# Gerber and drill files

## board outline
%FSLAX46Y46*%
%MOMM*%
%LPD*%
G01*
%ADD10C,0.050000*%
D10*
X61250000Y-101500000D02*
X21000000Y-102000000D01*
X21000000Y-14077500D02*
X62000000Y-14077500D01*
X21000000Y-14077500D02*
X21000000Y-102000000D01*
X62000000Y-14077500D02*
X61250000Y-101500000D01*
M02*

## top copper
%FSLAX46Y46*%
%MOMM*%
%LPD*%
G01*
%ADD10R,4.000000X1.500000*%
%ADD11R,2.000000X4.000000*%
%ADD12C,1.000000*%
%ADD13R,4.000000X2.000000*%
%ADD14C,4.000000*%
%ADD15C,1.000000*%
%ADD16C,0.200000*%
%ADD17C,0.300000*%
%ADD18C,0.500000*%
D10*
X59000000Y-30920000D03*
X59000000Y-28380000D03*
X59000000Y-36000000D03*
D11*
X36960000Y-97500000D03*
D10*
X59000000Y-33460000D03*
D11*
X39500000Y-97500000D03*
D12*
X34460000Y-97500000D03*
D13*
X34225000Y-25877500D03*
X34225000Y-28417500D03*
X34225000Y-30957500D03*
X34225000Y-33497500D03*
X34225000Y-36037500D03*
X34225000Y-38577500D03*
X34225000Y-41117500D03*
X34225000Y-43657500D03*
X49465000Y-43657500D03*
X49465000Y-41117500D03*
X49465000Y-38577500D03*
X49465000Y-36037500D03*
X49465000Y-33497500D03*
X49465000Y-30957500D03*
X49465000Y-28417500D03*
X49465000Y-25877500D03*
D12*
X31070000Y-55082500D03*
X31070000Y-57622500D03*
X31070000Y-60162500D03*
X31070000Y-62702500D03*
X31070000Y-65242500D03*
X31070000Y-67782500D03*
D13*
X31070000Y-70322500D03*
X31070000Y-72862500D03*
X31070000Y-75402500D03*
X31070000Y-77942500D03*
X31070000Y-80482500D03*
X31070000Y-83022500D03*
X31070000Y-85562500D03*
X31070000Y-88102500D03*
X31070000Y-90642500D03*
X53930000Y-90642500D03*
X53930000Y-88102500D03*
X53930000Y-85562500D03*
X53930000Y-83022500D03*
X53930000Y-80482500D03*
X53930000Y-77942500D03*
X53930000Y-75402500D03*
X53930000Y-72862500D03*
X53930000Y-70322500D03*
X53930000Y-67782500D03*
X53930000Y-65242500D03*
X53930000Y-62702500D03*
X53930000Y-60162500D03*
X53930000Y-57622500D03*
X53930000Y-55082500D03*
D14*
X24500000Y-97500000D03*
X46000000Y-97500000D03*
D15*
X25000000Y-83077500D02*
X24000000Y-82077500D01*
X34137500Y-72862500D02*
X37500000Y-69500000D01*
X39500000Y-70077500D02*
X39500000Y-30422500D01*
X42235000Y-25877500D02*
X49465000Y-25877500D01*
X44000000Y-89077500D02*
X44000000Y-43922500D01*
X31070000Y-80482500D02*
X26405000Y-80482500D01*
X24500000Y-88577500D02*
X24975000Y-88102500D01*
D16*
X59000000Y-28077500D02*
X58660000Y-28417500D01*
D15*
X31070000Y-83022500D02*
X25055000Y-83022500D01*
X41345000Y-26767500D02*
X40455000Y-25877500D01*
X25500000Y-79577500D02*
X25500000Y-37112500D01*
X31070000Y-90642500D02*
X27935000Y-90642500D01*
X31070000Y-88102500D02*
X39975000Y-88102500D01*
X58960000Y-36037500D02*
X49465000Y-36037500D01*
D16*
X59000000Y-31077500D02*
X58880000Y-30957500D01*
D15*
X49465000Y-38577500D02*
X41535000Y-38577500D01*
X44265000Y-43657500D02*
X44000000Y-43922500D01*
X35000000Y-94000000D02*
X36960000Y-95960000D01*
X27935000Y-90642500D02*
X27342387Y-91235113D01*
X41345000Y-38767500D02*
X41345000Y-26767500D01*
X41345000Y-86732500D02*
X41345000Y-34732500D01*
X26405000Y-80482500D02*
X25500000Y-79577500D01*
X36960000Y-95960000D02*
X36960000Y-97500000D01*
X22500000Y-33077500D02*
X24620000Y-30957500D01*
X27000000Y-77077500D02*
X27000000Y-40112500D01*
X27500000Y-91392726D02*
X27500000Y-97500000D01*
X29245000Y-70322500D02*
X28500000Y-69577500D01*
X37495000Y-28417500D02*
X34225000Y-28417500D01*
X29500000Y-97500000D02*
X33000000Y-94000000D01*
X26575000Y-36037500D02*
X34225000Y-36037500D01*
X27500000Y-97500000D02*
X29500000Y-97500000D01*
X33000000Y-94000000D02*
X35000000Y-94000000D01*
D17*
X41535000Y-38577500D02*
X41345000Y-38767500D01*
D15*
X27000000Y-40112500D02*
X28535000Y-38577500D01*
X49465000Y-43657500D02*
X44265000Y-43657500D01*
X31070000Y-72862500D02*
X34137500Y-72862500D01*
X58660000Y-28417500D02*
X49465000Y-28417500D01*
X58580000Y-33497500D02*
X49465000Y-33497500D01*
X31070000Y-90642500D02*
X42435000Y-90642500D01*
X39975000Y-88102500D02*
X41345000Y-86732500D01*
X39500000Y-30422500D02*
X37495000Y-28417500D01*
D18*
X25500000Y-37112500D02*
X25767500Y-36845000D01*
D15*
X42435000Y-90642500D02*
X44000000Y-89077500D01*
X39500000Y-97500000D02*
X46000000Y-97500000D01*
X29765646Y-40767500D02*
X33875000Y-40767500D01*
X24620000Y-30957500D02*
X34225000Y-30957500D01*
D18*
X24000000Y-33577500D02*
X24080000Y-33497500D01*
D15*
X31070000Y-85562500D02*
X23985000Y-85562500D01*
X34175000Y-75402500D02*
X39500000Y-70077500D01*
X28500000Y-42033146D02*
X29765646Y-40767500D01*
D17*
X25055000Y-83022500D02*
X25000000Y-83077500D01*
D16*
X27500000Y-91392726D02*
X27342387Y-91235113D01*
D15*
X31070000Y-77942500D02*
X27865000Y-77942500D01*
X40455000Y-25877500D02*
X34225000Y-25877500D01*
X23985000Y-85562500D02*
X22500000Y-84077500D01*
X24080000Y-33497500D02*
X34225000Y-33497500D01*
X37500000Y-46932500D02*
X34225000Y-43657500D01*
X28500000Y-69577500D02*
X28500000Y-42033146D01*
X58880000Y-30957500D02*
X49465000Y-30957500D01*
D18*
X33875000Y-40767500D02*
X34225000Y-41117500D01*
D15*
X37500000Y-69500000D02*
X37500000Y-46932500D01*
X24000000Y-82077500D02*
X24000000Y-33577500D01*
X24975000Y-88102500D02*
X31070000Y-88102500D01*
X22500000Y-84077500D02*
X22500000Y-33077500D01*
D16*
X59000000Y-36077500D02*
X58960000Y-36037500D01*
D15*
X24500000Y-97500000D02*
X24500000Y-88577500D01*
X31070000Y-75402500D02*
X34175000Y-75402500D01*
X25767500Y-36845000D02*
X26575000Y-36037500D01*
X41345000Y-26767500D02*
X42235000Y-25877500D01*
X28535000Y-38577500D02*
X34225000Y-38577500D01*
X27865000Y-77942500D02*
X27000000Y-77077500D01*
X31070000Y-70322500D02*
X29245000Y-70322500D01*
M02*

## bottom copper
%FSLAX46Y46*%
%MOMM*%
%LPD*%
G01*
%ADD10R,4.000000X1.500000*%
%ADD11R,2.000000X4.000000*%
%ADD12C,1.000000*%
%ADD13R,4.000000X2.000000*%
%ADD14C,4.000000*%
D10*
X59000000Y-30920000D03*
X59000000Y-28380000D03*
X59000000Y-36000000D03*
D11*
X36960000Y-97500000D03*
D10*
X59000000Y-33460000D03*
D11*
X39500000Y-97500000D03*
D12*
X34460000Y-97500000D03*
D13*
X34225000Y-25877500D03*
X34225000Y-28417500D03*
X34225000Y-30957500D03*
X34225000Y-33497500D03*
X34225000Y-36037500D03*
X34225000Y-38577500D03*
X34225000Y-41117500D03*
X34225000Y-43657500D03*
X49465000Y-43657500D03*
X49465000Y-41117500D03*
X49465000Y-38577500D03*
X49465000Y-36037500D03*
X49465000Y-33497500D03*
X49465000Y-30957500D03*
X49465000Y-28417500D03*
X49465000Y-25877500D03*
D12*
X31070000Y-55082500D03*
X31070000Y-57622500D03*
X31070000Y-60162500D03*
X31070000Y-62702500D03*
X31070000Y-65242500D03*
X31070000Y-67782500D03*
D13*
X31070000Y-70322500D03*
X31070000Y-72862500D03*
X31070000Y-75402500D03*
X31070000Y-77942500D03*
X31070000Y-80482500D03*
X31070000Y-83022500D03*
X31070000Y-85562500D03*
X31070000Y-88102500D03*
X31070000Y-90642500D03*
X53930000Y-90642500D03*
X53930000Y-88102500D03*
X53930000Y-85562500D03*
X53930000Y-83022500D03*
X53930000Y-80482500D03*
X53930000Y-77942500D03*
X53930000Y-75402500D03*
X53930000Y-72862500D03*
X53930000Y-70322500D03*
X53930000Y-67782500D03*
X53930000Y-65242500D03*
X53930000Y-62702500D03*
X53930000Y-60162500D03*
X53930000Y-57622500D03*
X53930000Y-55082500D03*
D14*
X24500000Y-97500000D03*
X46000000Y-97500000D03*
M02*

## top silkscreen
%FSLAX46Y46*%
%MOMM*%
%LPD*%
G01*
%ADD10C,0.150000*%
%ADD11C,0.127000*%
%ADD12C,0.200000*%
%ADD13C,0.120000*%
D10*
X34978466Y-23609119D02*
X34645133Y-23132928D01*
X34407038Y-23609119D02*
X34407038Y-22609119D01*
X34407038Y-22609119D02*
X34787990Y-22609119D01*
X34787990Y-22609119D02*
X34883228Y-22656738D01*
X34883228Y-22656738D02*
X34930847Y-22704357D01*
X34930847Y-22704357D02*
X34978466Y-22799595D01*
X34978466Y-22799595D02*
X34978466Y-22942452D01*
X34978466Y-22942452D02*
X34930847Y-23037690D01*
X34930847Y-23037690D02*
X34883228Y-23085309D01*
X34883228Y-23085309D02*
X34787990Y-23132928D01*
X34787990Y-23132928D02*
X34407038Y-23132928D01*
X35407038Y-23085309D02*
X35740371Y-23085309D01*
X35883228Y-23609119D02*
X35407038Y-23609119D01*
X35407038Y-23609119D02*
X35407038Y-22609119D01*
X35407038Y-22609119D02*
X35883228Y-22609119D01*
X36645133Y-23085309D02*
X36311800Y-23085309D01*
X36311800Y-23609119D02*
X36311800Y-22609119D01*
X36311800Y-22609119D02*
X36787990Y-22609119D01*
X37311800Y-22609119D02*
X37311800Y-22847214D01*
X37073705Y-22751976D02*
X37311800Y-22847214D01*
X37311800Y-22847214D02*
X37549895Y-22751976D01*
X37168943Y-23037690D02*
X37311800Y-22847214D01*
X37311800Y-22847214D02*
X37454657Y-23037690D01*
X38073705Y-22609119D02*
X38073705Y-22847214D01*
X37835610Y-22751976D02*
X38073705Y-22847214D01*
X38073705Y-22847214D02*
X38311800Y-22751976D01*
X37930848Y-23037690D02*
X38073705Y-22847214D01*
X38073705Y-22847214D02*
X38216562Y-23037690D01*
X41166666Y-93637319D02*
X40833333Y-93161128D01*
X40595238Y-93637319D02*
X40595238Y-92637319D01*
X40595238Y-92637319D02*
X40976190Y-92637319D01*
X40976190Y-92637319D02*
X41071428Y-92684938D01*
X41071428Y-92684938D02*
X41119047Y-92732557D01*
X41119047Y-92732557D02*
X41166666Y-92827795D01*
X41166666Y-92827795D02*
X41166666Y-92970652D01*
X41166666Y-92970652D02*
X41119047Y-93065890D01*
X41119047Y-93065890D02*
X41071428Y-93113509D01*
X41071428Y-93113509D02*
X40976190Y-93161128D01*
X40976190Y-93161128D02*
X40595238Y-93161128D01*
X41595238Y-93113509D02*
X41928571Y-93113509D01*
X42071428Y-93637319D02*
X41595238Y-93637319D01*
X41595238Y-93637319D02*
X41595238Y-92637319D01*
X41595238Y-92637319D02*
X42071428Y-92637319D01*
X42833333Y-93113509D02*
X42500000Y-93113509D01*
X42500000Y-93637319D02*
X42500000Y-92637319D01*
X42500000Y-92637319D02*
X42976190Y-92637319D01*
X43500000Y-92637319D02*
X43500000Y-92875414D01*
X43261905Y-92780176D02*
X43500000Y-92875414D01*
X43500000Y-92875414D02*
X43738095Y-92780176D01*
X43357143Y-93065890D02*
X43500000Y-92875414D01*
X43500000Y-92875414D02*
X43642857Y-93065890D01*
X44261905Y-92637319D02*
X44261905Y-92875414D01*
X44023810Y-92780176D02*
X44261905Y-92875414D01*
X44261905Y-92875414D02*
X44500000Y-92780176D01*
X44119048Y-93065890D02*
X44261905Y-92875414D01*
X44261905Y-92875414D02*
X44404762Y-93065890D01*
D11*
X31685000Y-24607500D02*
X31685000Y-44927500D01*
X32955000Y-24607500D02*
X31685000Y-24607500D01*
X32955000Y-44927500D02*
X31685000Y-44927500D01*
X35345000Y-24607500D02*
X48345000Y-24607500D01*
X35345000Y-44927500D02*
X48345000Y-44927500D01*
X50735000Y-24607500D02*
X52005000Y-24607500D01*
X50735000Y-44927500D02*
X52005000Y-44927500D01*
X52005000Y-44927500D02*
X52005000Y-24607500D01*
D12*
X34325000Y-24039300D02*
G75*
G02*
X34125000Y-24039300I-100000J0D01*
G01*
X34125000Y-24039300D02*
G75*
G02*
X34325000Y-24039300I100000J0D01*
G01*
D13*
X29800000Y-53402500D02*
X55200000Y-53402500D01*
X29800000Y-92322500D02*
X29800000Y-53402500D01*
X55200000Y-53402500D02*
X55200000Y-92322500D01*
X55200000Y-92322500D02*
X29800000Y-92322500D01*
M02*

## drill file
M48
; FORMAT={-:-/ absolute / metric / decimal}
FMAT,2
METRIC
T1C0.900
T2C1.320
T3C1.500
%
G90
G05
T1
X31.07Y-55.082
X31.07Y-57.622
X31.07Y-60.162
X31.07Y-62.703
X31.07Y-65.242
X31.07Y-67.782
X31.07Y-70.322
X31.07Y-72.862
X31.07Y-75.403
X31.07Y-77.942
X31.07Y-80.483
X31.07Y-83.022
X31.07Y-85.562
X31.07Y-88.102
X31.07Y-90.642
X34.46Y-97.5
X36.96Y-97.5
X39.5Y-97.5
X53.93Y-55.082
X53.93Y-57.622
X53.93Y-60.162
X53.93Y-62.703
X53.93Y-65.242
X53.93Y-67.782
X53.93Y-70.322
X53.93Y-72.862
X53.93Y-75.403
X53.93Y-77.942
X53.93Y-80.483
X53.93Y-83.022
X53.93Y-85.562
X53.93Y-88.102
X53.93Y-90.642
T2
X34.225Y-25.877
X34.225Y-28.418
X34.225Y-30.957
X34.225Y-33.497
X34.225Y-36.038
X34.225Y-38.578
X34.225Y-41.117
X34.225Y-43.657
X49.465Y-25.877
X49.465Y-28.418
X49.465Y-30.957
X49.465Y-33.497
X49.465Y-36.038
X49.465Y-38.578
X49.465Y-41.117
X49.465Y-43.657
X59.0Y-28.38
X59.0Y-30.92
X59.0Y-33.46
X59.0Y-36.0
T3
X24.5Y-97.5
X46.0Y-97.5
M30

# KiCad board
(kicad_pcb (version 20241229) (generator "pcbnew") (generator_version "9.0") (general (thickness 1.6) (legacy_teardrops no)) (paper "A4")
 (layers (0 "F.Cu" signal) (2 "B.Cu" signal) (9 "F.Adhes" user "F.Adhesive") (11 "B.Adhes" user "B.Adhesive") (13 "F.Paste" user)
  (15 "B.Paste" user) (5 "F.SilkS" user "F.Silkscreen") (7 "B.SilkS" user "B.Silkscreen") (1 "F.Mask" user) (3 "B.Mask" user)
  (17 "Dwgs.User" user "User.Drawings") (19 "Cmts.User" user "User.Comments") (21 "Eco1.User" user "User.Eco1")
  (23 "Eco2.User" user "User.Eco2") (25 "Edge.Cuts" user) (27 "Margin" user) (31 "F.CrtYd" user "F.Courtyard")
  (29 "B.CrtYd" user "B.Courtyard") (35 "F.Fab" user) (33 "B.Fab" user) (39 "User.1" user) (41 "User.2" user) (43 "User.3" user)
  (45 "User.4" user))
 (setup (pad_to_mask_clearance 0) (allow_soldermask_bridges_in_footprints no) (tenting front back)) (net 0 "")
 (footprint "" (layer "F.Cu") (at 59 30.92)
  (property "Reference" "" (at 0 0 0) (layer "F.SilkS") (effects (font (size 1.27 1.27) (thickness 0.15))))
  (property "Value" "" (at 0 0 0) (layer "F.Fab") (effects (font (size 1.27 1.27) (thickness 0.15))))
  (pad "14" thru_hole rect (at 0 0) (size 4 1.5) (drill 1.32) (layers "*.Cu" "*.Mask") (remove_unused_layers no) (solder_mask_margin 0.102)))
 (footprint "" (layer "F.Cu") (at 59 28.38)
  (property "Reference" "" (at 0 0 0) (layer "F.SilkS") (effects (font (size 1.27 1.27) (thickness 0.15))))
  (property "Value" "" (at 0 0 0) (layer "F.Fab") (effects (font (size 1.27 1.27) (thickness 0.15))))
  (pad "15" thru_hole rect (at 0 0) (size 4 1.5) (drill 1.32) (layers "*.Cu" "*.Mask") (remove_unused_layers no) (solder_mask_margin 0.102)))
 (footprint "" (layer "F.Cu") (at 59 36)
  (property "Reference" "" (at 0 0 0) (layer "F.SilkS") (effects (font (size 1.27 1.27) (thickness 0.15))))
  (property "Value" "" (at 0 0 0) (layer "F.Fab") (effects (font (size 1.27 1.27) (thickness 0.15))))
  (pad "12" thru_hole rect (at 0 0) (size 4 1.5) (drill 1.32) (layers "*.Cu" "*.Mask") (remove_unused_layers no) (solder_mask_margin 0.102)))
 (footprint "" (layer "F.Cu") (at 36.96 97.5 -90)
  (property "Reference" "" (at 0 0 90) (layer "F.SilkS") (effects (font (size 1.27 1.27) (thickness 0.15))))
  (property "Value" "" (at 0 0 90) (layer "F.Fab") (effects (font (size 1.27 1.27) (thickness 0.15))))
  (pad "17" thru_hole rect (at 0 0 270) (size 4 2) (drill 0.9) (layers "*.Cu" "*.Mask") (remove_unused_layers yes) (keep_end_layers yes)
   (zone_layer_connections) (thermal_bridge_width 2) (thermal_gap 4)))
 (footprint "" (layer "F.Cu") (at 59 33.46)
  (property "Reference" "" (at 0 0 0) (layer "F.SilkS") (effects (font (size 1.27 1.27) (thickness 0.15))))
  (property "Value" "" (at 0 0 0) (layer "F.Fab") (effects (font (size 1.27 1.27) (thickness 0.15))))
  (pad "13" thru_hole rect (at 0 0) (size 4 1.5) (drill 1.32) (layers "*.Cu" "*.Mask") (remove_unused_layers no) (solder_mask_margin 0.102)))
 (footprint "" (layer "F.Cu") (at 39.5 97.5)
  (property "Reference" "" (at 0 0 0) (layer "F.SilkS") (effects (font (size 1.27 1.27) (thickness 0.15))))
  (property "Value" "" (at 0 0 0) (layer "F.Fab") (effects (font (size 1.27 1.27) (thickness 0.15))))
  (pad "18" thru_hole rect (at 0 0 270) (size 4 2) (drill 0.9) (layers "*.Cu" "*.Mask") (remove_unused_layers yes) (keep_end_layers yes)
   (zone_layer_connections)))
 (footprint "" (layer "F.Cu") (at 34.46 97.5 -90)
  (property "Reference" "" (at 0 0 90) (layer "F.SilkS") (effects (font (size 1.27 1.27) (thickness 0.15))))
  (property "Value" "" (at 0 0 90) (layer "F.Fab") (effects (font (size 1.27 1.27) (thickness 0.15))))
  (pad "17" thru_hole circle (at 0 0 270) (size 1 1) (drill 0.9) (layers "*.Cu" "*.Mask") (remove_unused_layers yes) (keep_end_layers yes)
   (zone_layer_connections) (thermal_bridge_width 2) (thermal_gap 4)))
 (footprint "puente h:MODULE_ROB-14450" (layer "F.Cu") (at 41.845 34.7675)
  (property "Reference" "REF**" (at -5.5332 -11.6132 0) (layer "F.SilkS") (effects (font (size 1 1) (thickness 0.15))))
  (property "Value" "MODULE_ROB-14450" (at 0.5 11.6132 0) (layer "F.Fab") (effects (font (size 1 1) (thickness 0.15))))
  (fp_line (start -10.16 -10.16) (end -10.16 10.16) (stroke (width 0.127) (type solid)) (layer "F.SilkS"))
  (fp_line (start -8.89 -10.16) (end -10.16 -10.16) (stroke (width 0.127) (type solid)) (layer "F.SilkS"))
  (fp_line (start -8.89 10.16) (end -10.16 10.16) (stroke (width 0.127) (type solid)) (layer "F.SilkS"))
  (fp_line (start -6.5 -10.16) (end 6.5 -10.16) (stroke (width 0.127) (type solid)) (layer "F.SilkS"))
  (fp_line (start -6.5 10.16) (end 6.5 10.16) (stroke (width 0.127) (type solid)) (layer "F.SilkS"))
  (fp_line (start 8.89 -10.16) (end 10.16 -10.16) (stroke (width 0.127) (type solid)) (layer "F.SilkS"))
  (fp_line (start 8.89 10.16) (end 10.16 10.16) (stroke (width 0.127) (type solid)) (layer "F.SilkS"))
  (fp_line (start 10.16 10.16) (end 10.16 -10.16) (stroke (width 0.127) (type solid)) (layer "F.SilkS"))
  (fp_circle (center -7.62 -10.7282) (end -7.52 -10.7282) (stroke (width 0.2) (type solid)) (fill no) (layer "F.SilkS"))
  (pad "1" thru_hole rect (at -7.62 -8.89) (size 4 2) (drill 1.32) (layers "*.Cu" "*.Mask") (remove_unused_layers no)
   (solder_mask_margin 0.102))
  (pad "2" thru_hole rect (at -7.62 -6.35) (size 4 2) (drill 1.32) (layers "*.Cu" "*.Mask") (remove_unused_layers no)
   (solder_mask_margin 0.102))
  (pad "3" thru_hole rect (at -7.62 -3.81) (size 4 2) (drill 1.32) (layers "*.Cu" "*.Mask") (remove_unused_layers no)
   (solder_mask_margin 0.102))
  (pad "4" thru_hole rect (at -7.62 -1.27) (size 4 2) (drill 1.32) (layers "*.Cu" "*.Mask") (remove_unused_layers no)
   (solder_mask_margin 0.102))
  (pad "5" thru_hole rect (at -7.62 1.27) (size 4 2) (drill 1.32) (layers "*.Cu" "*.Mask") (remove_unused_layers no)
   (solder_mask_margin 0.102))
  (pad "6" thru_hole rect (at -7.62 3.81) (size 4 2) (drill 1.32) (layers "*.Cu" "*.Mask") (remove_unused_layers no)
   (solder_mask_margin 0.102))
  (pad "7" thru_hole rect (at -7.62 6.35) (size 4 2) (drill 1.32) (layers "*.Cu" "*.Mask") (remove_unused_layers no)
   (solder_mask_margin 0.102))
  (pad "8" thru_hole rect (at -7.62 8.89) (size 4 2) (drill 1.32) (layers "*.Cu" "*.Mask") (remove_unused_layers no)
   (solder_mask_margin 0.102))
  (pad "9" thru_hole rect (at 7.62 8.89) (size 4 2) (drill 1.32) (layers "*.Cu" "*.Mask") (remove_unused_layers no)
   (solder_mask_margin 0.102))
  (pad "10" thru_hole rect (at 7.62 6.35) (size 4 2) (drill 1.32) (layers "*.Cu" "*.Mask") (remove_unused_layers no)
   (solder_mask_margin 0.102))
  (pad "11" thru_hole rect (at 7.62 3.81) (size 4 2) (drill 1.32) (layers "*.Cu" "*.Mask") (remove_unused_layers no)
   (solder_mask_margin 0.102))
  (pad "12" thru_hole rect (at 7.62 1.27) (size 4 2) (drill 1.32) (layers "*.Cu" "*.Mask") (remove_unused_layers no)
   (solder_mask_margin 0.102))
  (pad "13" thru_hole rect (at 7.62 -1.27) (size 4 2) (drill 1.32) (layers "*.Cu" "*.Mask") (remove_unused_layers no)
   (solder_mask_margin 0.102))
  (pad "14" thru_hole rect (at 7.62 -3.81) (size 4 2) (drill 1.32) (layers "*.Cu" "*.Mask") (remove_unused_layers no)
   (solder_mask_margin 0.102))
  (pad "15" thru_hole rect (at 7.62 -6.35) (size 4 2) (drill 1.32) (layers "*.Cu" "*.Mask") (remove_unused_layers no)
   (solder_mask_margin 0.102))
  (pad "16" thru_hole rect (at 7.62 -8.89) (size 4 2) (drill 1.32) (layers "*.Cu" "*.Mask") (remove_unused_layers no)
   (solder_mask_margin 0.102)))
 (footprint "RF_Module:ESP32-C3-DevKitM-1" (layer "F.Cu") (at 31.07 55.0825)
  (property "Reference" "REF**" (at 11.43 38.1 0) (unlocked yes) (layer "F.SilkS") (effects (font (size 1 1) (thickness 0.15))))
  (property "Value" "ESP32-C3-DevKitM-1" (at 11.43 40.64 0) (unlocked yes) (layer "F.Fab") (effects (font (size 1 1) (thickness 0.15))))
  (fp_line (start -1.27 -1.68) (end 24.13 -1.68) (stroke (width 0.12) (type solid)) (layer "F.SilkS"))
  (fp_line (start -1.27 37.24) (end -1.27 -1.68) (stroke (width 0.12) (type solid)) (layer "F.SilkS"))
  (fp_line (start 24.13 -1.68) (end 24.13 37.24) (stroke (width 0.12) (type solid)) (layer "F.SilkS"))
  (fp_line (start 24.13 37.24) (end -1.27 37.24) (stroke (width 0.12) (type solid)) (layer "F.SilkS"))
  (pad "1" thru_hole circle (at 0 0) (size 1 1) (drill 0.9) (layers "*.Cu" "*.Mask") (remove_unused_layers yes) (keep_end_layers yes)
   (zone_layer_connections) (thermal_bridge_width 2) (thermal_gap 4))
  (pad "2" thru_hole circle (at 0 2.54) (size 1 1) (drill 0.9) (layers "*.Cu" "*.Mask") (remove_unused_layers yes) (keep_end_layers yes)
   (zone_layer_connections) (thermal_bridge_width 2) (thermal_gap 4))
  (pad "3" thru_hole circle (at 0 5.08) (size 1 1) (drill 0.9) (layers "*.Cu" "*.Mask") (remove_unused_layers yes) (keep_end_layers yes)
   (zone_layer_connections) (thermal_bridge_width 2) (thermal_gap 4))
  (pad "4" thru_hole circle (at 0 7.62) (size 1 1) (drill 0.9) (layers "*.Cu" "*.Mask") (remove_unused_layers yes) (keep_end_layers yes)
   (zone_layer_connections) (thermal_bridge_width 2) (thermal_gap 4))
  (pad "5" thru_hole circle (at 0 10.16) (size 1 1) (drill 0.9) (layers "*.Cu" "*.Mask") (remove_unused_layers yes) (keep_end_layers yes)
   (zone_layer_connections) (thermal_bridge_width 2) (thermal_gap 4))
  (pad "6" thru_hole circle (at 0 12.7) (size 1 1) (drill 0.9) (layers "*.Cu" "*.Mask") (remove_unused_layers yes) (keep_end_layers yes)
   (zone_layer_connections) (thermal_bridge_width 2) (thermal_gap 4))
  (pad "7" thru_hole rect (at 0 15.24) (size 4 2) (drill 0.9) (layers "*.Cu" "*.Mask") (remove_unused_layers yes) (keep_end_layers yes)
   (zone_layer_connections) (thermal_bridge_width 2) (thermal_gap 4))
  (pad "8" thru_hole rect (at 0 17.78) (size 4 2) (drill 0.9) (layers "*.Cu" "*.Mask") (remove_unused_layers yes) (keep_end_layers yes)
   (zone_layer_connections) (thermal_bridge_width 2) (thermal_gap 4))
  (pad "9" thru_hole rect (at 0 20.32) (size 4 2) (drill 0.9) (layers "*.Cu" "*.Mask") (remove_unused_layers yes) (keep_end_layers yes)
   (zone_layer_connections) (thermal_bridge_width 2) (thermal_gap 4))
  (pad "10" thru_hole rect (at 0 22.86) (size 4 2) (drill 0.9) (layers "*.Cu" "*.Mask") (remove_unused_layers yes) (keep_end_layers yes)
   (zone_layer_connections) (thermal_bridge_width 2) (thermal_gap 4))
  (pad "11" thru_hole rect (at 0 25.4) (size 4 2) (drill 0.9) (layers "*.Cu" "*.Mask") (remove_unused_layers yes) (keep_end_layers yes)
   (zone_layer_connections) (thermal_bridge_width 2) (thermal_gap 4))
  (pad "12" thru_hole rect (at 0 27.94) (size 4 2) (drill 0.9) (layers "*.Cu" "*.Mask") (remove_unused_layers yes) (keep_end_layers yes)
   (zone_layer_connections) (thermal_bridge_width 2) (thermal_gap 4))
  (pad "13" thru_hole rect (at 0 30.48) (size 4 2) (drill 0.9) (layers "*.Cu" "*.Mask") (remove_unused_layers yes) (keep_end_layers yes)
   (zone_layer_connections) (thermal_bridge_width 2) (thermal_gap 4))
  (pad "14" thru_hole rect (at 0 33.02) (size 4 2) (drill 0.9) (layers "*.Cu" "*.Mask") (remove_unused_layers yes) (keep_end_layers yes)
   (zone_layer_connections) (thermal_bridge_width 2) (thermal_gap 4))
  (pad "15" thru_hole rect (at 0 35.56) (size 4 2) (drill 0.9) (layers "*.Cu" "*.Mask") (remove_unused_layers yes) (keep_end_layers yes)
   (zone_layer_connections) (thermal_bridge_width 2) (thermal_gap 4))
  (pad "16" thru_hole rect (at 22.86 35.56) (size 4 2) (drill 0.9) (layers "*.Cu" "*.Mask") (remove_unused_layers yes) (keep_end_layers yes)
   (zone_layer_connections) (thermal_bridge_width 2) (thermal_gap 4))
  (pad "17" thru_hole rect (at 22.86 33.02) (size 4 2) (drill 0.9) (layers "*.Cu" "*.Mask") (remove_unused_layers yes) (keep_end_layers yes)
   (zone_layer_connections) (thermal_bridge_width 2) (thermal_gap 4))
  (pad "18" thru_hole rect (at 22.86 30.48) (size 4 2) (drill 0.9) (layers "*.Cu" "*.Mask") (remove_unused_layers yes) (keep_end_layers yes)
   (zone_layer_connections) (thermal_bridge_width 2) (thermal_gap 4))
  (pad "19" thru_hole rect (at 22.86 27.94) (size 4 2) (drill 0.9) (layers "*.Cu" "*.Mask") (remove_unused_layers yes) (keep_end_layers yes)
   (zone_layer_connections) (thermal_bridge_width 2) (thermal_gap 4))
  (pad "20" thru_hole rect (at 22.86 25.4) (size 4 2) (drill 0.9) (layers "*.Cu" "*.Mask") (remove_unused_layers yes) (keep_end_layers yes)
   (zone_layer_connections) (thermal_bridge_width 2) (thermal_gap 4))
  (pad "21" thru_hole rect (at 22.86 22.86) (size 4 2) (drill 0.9) (layers "*.Cu" "*.Mask") (remove_unused_layers yes) (keep_end_layers yes)
   (zone_layer_connections) (thermal_bridge_width 2) (thermal_gap 4))
  (pad "22" thru_hole rect (at 22.86 20.32) (size 4 2) (drill 0.9) (layers "*.Cu" "*.Mask") (remove_unused_layers yes) (keep_end_layers yes)
   (zone_layer_connections) (thermal_bridge_width 2) (thermal_gap 4))
  (pad "23" thru_hole rect (at 22.86 17.78) (size 4 2) (drill 0.9) (layers "*.Cu" "*.Mask") (remove_unused_layers yes) (keep_end_layers yes)
   (zone_layer_connections) (thermal_bridge_width 2) (thermal_gap 4))
  (pad "24" thru_hole rect (at 22.86 15.24) (size 4 2) (drill 0.9) (layers "*.Cu" "*.Mask") (remove_unused_layers yes) (keep_end_layers yes)
   (zone_layer_connections) (thermal_bridge_width 2) (thermal_gap 4))
  (pad "25" thru_hole rect (at 22.86 12.7) (size 4 2) (drill 0.9) (layers "*.Cu" "*.Mask") (remove_unused_layers yes) (keep_end_layers yes)
   (zone_layer_connections) (thermal_bridge_width 2) (thermal_gap 4))
  (pad "26" thru_hole rect (at 22.86 10.16) (size 4 2) (drill 0.9) (layers "*.Cu" "*.Mask") (remove_unused_layers yes) (keep_end_layers yes)
   (zone_layer_connections) (thermal_bridge_width 2) (thermal_gap 4))
  (pad "27" thru_hole rect (at 22.86 7.62) (size 4 2) (drill 0.9) (layers "*.Cu" "*.Mask") (remove_unused_layers yes) (keep_end_layers yes)
   (zone_layer_connections) (thermal_bridge_width 2) (thermal_gap 4))
  (pad "28" thru_hole rect (at 22.86 5.08) (size 4 2) (drill 0.9) (layers "*.Cu" "*.Mask") (remove_unused_layers yes) (keep_end_layers yes)
   (zone_layer_connections) (thermal_bridge_width 2) (thermal_gap 4))
  (pad "29" thru_hole rect (at 22.86 2.54) (size 4 2) (drill 0.9) (layers "*.Cu" "*.Mask") (remove_unused_layers yes) (keep_end_layers yes)
   (zone_layer_connections) (thermal_bridge_width 2) (thermal_gap 4))
  (pad "30" thru_hole rect (at 22.86 0) (size 4 2) (drill 0.9) (layers "*.Cu" "*.Mask") (remove_unused_layers yes) (keep_end_layers yes)
   (zone_layer_connections) (thermal_bridge_width 2) (thermal_gap 4)))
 (gr_line (start 61.25 101.5) (end 21 102) (stroke (width 0.05) (type default)) (layer "Edge.Cuts"))
 (gr_line (start 21 14.0775) (end 62 14.0775) (stroke (width 0.05) (type default)) (layer "Edge.Cuts"))
 (gr_line (start 21 14.0775) (end 21 102) (stroke (width 0.05) (type default)) (layer "Edge.Cuts"))
 (gr_line (start 62 14.0775) (end 61.25 101.5) (stroke (width 0.05) (type default)) (layer "Edge.Cuts"))
 (segment (start 25 83.0775) (end 24 82.0775) (width 1) (layer "F.Cu") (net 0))
 (segment (start 34.1375 72.8625) (end 37.5 69.5) (width 1) (layer "F.Cu") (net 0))
 (segment (start 39.5 70.0775) (end 39.5 30.4225) (width 1) (layer "F.Cu") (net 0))
 (segment (start 42.235 25.8775) (end 49.465 25.8775) (width 1) (layer "F.Cu") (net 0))
 (segment (start 44 89.0775) (end 44 43.9225) (width 1) (layer "F.Cu") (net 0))
 (segment (start 31.07 80.4825) (end 26.405 80.4825) (width 1) (layer "F.Cu") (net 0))
 (segment (start 24.5 88.5775) (end 24.975 88.1025) (width 1) (layer "F.Cu") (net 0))
 (segment (start 59 28.0775) (end 58.66 28.4175) (width 0.2) (layer "F.Cu") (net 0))
 (segment (start 31.07 83.0225) (end 25.055 83.0225) (width 1) (layer "F.Cu") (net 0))
 (segment (start 41.345 26.7675) (end 40.455 25.8775) (width 1) (layer "F.Cu") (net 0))
 (segment (start 25.5 79.5775) (end 25.5 37.1125) (width 1) (layer "F.Cu") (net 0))
 (segment (start 31.07 90.6425) (end 27.935 90.6425) (width 1) (layer "F.Cu") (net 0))
 (segment (start 31.07 88.1025) (end 39.975 88.1025) (width 1) (layer "F.Cu") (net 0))
 (segment (start 58.96 36.0375) (end 49.465 36.0375) (width 1) (layer "F.Cu") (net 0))
 (segment (start 59 31.0775) (end 58.88 30.9575) (width 0.2) (layer "F.Cu") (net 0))
 (segment (start 49.465 38.5775) (end 41.535 38.5775) (width 1) (layer "F.Cu") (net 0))
 (segment (start 44.265 43.6575) (end 44 43.9225) (width 1) (layer "F.Cu") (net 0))
 (segment (start 35 94) (end 36.96 95.96) (width 1) (layer "F.Cu") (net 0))
 (segment (start 27.935 90.6425) (end 27.342387 91.235113) (width 1) (layer "F.Cu") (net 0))
 (segment (start 41.345 38.7675) (end 41.345 26.7675) (width 1) (layer "F.Cu") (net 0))
 (segment (start 41.345 86.7325) (end 41.345 34.7325) (width 1) (layer "F.Cu") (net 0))
 (segment (start 26.405 80.4825) (end 25.5 79.5775) (width 1) (layer "F.Cu") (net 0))
 (segment (start 36.96 95.96) (end 36.96 97.5) (width 1) (layer "F.Cu") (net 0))
 (segment (start 22.5 33.0775) (end 24.62 30.9575) (width 1) (layer "F.Cu") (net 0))
 (segment (start 27 77.0775) (end 27 40.1125) (width 1) (layer "F.Cu") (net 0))
 (segment (start 27.5 91.392726) (end 27.5 97.5) (width 1) (layer "F.Cu") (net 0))
 (segment (start 29.245 70.3225) (end 28.5 69.5775) (width 1) (layer "F.Cu") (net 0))
 (segment (start 37.495 28.4175) (end 34.225 28.4175) (width 1) (layer "F.Cu") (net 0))
 (segment (start 29.5 97.5) (end 33 94) (width 1) (layer "F.Cu") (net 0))
 (segment (start 26.575 36.0375) (end 34.225 36.0375) (width 1) (layer "F.Cu") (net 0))
 (segment (start 27.5 97.5) (end 29.5 97.5) (width 1) (layer "F.Cu") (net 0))
 (segment (start 33 94) (end 35 94) (width 1) (layer "F.Cu") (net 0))
 (segment (start 41.535 38.5775) (end 41.345 38.7675) (width 0.3) (layer "F.Cu") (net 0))
 (segment (start 27 40.1125) (end 28.535 38.5775) (width 1) (layer "F.Cu") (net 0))
 (segment (start 49.465 43.6575) (end 44.265 43.6575) (width 1) (layer "F.Cu") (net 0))
 (segment (start 31.07 72.8625) (end 34.1375 72.8625) (width 1) (layer "F.Cu") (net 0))
 (segment (start 58.66 28.4175) (end 49.465 28.4175) (width 1) (layer "F.Cu") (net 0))
 (segment (start 58.58 33.4975) (end 49.465 33.4975) (width 1) (layer "F.Cu") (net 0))
 (segment (start 31.07 90.6425) (end 42.435 90.6425) (width 1) (layer "F.Cu") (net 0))
 (segment (start 39.975 88.1025) (end 41.345 86.7325) (width 1) (layer "F.Cu") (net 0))
 (segment (start 39.5 30.4225) (end 37.495 28.4175) (width 1) (layer "F.Cu") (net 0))
 (segment (start 25.5 37.1125) (end 25.7675 36.845) (width 0.5) (layer "F.Cu") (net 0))
 (segment (start 42.435 90.6425) (end 44 89.0775) (width 1) (layer "F.Cu") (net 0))
 (segment (start 39.5 97.5) (end 46 97.5) (width 1) (layer "F.Cu") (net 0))
 (segment (start 29.765646 40.7675) (end 33.875 40.7675) (width 1) (layer "F.Cu") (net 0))
 (segment (start 24.62 30.9575) (end 34.225 30.9575) (width 1) (layer "F.Cu") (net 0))
 (segment (start 24 33.5775) (end 24.08 33.4975) (width 0.5) (layer "F.Cu") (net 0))
 (segment (start 31.07 85.5625) (end 23.985 85.5625) (width 1) (layer "F.Cu") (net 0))
 (segment (start 34.175 75.4025) (end 39.5 70.0775) (width 1) (layer "F.Cu") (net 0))
 (segment (start 28.5 42.033146) (end 29.765646 40.7675) (width 1) (layer "F.Cu") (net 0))
 (segment (start 25.055 83.0225) (end 25 83.0775) (width 0.3) (layer "F.Cu") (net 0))
 (segment (start 27.5 91.392726) (end 27.342387 91.235113) (width 0.2) (layer "F.Cu") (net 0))
 (segment (start 31.07 77.9425) (end 27.865 77.9425) (width 1) (layer "F.Cu") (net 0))
 (segment (start 40.455 25.8775) (end 34.225 25.8775) (width 1) (layer "F.Cu") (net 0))
 (segment (start 23.985 85.5625) (end 22.5 84.0775) (width 1) (layer "F.Cu") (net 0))
 (segment (start 24.08 33.4975) (end 34.225 33.4975) (width 1) (layer "F.Cu") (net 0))
 (segment (start 37.5 46.9325) (end 34.225 43.6575) (width 1) (layer "F.Cu") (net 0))
 (segment (start 28.5 69.5775) (end 28.5 42.033146) (width 1) (layer "F.Cu") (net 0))
 (segment (start 58.88 30.9575) (end 49.465 30.9575) (width 1) (layer "F.Cu") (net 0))
 (segment (start 33.875 40.7675) (end 34.225 41.1175) (width 0.5) (layer "F.Cu") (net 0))
 (segment (start 37.5 69.5) (end 37.5 46.9325) (width 1) (layer "F.Cu") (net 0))
 (segment (start 24 82.0775) (end 24 33.5775) (width 1) (layer "F.Cu") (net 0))
 (segment (start 24.975 88.1025) (end 31.07 88.1025) (width 1) (layer "F.Cu") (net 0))
 (segment (start 22.5 84.0775) (end 22.5 33.0775) (width 1) (layer "F.Cu") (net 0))
 (segment (start 59 36.0775) (end 58.96 36.0375) (width 0.2) (layer "F.Cu") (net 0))
 (segment (start 24.5 97.5) (end 24.5 88.5775) (width 1) (layer "F.Cu") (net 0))
 (segment (start 31.07 75.4025) (end 34.175 75.4025) (width 1) (layer "F.Cu") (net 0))
 (segment (start 25.7675 36.845) (end 26.575 36.0375) (width 1) (layer "F.Cu") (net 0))
 (segment (start 41.345 26.7675) (end 42.235 25.8775) (width 1) (layer "F.Cu") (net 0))
 (segment (start 28.535 38.5775) (end 34.225 38.5775) (width 1) (layer "F.Cu") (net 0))
 (segment (start 27.865 77.9425) (end 27 77.0775) (width 1) (layer "F.Cu") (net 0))
 (segment (start 31.07 70.3225) (end 29.245 70.3225) (width 1) (layer "F.Cu") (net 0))
 (via (at 24.5 97.5) (size 4) (drill 1.5) (layers "F.Cu" "B.Cu") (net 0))
 (via (at 46 97.5) (size 4) (drill 1.5) (layers "F.Cu" "B.Cu")
  (teardrops (best_length_ratio 1) (max_length 2) (best_width_ratio 2) (max_width 5) (curved_edges no) (filter_ratio 0.9) (enabled no)
   (allow_two_segments yes) (prefer_zone_connections yes))
  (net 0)))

